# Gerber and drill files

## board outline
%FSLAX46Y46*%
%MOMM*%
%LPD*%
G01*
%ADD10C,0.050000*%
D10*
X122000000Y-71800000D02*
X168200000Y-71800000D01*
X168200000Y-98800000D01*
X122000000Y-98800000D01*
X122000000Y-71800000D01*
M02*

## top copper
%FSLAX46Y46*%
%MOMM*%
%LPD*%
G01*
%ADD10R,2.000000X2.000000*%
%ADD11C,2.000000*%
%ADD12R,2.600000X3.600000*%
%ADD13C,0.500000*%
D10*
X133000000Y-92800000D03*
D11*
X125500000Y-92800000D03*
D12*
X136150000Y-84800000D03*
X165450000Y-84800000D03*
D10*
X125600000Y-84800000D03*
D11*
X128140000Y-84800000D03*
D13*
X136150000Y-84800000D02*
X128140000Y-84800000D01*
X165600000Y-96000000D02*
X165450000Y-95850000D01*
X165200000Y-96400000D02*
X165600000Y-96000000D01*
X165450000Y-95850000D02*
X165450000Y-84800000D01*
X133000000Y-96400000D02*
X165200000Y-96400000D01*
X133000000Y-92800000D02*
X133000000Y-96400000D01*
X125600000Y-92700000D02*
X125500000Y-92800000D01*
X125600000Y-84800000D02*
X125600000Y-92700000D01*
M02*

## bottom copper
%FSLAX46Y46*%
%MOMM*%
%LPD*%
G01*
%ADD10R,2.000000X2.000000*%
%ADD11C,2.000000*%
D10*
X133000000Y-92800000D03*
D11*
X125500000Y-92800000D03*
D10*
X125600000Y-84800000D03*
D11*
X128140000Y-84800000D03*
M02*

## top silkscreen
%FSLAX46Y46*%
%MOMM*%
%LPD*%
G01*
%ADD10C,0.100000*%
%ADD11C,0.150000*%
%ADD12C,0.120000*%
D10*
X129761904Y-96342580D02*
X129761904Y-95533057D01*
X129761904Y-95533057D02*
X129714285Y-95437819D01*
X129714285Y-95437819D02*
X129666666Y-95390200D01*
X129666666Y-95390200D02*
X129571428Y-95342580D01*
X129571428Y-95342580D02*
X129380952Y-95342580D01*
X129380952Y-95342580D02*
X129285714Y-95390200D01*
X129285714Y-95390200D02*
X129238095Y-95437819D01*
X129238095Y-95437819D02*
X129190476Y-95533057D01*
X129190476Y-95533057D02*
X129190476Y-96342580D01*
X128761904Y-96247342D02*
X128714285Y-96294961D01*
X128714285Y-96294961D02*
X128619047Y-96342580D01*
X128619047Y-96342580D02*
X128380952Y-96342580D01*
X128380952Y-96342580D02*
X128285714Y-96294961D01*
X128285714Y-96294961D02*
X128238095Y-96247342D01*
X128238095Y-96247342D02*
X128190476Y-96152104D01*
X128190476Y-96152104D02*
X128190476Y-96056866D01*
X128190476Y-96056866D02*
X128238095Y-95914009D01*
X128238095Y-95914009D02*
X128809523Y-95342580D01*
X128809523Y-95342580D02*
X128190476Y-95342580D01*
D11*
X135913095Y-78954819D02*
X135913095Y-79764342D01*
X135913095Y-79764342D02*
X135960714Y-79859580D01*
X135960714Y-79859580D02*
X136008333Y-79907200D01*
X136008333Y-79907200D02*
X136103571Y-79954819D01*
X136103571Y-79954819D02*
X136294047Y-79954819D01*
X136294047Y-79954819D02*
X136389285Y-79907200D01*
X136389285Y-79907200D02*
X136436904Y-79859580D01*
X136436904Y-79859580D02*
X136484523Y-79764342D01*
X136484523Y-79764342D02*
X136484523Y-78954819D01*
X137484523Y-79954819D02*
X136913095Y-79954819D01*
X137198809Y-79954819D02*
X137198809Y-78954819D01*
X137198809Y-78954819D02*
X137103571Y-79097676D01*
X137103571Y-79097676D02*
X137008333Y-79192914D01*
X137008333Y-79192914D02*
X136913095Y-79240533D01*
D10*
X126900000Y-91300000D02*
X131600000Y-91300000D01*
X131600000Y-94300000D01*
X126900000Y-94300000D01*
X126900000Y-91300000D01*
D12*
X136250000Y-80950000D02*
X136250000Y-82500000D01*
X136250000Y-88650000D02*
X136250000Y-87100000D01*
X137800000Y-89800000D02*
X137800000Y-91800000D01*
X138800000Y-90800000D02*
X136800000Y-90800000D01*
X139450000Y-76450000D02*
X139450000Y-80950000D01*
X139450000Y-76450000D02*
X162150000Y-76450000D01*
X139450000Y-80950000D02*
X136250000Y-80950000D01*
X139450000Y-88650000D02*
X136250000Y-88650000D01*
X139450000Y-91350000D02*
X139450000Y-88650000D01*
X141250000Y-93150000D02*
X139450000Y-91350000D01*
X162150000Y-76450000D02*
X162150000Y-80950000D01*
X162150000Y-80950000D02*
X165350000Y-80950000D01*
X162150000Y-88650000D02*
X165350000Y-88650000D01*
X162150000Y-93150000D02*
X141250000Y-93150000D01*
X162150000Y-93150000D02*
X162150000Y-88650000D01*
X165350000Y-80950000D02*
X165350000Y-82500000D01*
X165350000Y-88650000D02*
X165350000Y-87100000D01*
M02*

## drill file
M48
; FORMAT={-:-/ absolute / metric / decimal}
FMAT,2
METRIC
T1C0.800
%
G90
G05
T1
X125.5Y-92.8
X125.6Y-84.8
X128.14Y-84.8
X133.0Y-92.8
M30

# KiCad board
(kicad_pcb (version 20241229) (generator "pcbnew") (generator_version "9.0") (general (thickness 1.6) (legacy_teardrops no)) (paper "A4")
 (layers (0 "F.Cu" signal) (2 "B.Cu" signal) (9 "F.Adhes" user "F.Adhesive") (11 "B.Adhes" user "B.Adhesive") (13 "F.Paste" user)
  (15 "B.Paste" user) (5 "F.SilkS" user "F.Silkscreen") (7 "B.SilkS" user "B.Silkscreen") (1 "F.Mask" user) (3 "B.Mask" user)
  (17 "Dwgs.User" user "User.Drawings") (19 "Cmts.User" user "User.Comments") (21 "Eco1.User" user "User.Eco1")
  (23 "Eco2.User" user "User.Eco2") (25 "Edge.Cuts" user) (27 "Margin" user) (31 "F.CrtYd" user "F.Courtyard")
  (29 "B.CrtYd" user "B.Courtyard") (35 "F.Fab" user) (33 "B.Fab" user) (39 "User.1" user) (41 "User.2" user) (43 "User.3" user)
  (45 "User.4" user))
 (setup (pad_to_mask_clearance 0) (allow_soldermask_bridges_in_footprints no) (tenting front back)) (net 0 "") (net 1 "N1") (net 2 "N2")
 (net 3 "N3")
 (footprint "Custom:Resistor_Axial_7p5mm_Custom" (layer "F.Cu") (at 133 92.8 180)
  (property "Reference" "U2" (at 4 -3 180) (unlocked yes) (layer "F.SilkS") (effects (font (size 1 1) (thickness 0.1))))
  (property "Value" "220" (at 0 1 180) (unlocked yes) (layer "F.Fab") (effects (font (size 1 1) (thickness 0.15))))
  (fp_rect (start 1.4 -1.5) (end 6.1 1.5) (stroke (width 0.1) (type solid)) (fill no) (layer "F.SilkS"))
  (pad "1" thru_hole rect (at 0 0 180) (size 2 2) (drill 0.8) (layers "*.Cu" "*.Mask") (remove_unused_layers no) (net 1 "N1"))
  (pad "2" thru_hole circle (at 7.5 0 180) (size 2 2) (drill 0.8) (layers "*.Cu" "*.Mask") (remove_unused_layers no) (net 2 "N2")))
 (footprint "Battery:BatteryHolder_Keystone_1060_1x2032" (layer "F.Cu") (at 150.8 84.8)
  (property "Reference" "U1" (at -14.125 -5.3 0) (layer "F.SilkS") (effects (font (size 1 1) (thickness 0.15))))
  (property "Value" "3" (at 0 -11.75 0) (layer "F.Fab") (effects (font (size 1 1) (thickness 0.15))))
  (fp_line (start -14.55 -3.85) (end -14.55 -2.3) (stroke (width 0.12) (type solid)) (layer "F.SilkS"))
  (fp_line (start -14.55 3.85) (end -14.55 2.3) (stroke (width 0.12) (type solid)) (layer "F.SilkS"))
  (fp_line (start -13 5) (end -13 7) (stroke (width 0.12) (type solid)) (layer "F.SilkS"))
  (fp_line (start -12 6) (end -14 6) (stroke (width 0.12) (type solid)) (layer "F.SilkS"))
  (fp_line (start -11.35 -8.35) (end -11.35 -3.85) (stroke (width 0.12) (type solid)) (layer "F.SilkS"))
  (fp_line (start -11.35 -8.35) (end 11.35 -8.35) (stroke (width 0.12) (type solid)) (layer "F.SilkS"))
  (fp_line (start -11.35 -3.85) (end -14.55 -3.85) (stroke (width 0.12) (type solid)) (layer "F.SilkS"))
  (fp_line (start -11.35 3.85) (end -14.55 3.85) (stroke (width 0.12) (type solid)) (layer "F.SilkS"))
  (fp_line (start -11.35 6.55) (end -11.35 3.85) (stroke (width 0.12) (type solid)) (layer "F.SilkS"))
  (fp_line (start -9.55 8.35) (end -11.35 6.55) (stroke (width 0.12) (type solid)) (layer "F.SilkS"))
  (fp_line (start 11.35 -8.35) (end 11.35 -3.85) (stroke (width 0.12) (type solid)) (layer "F.SilkS"))
  (fp_line (start 11.35 -3.85) (end 14.55 -3.85) (stroke (width 0.12) (type solid)) (layer "F.SilkS"))
  (fp_line (start 11.35 3.85) (end 14.55 3.85) (stroke (width 0.12) (type solid)) (layer "F.SilkS"))
  (fp_line (start 11.35 8.35) (end -9.55 8.35) (stroke (width 0.12) (type solid)) (layer "F.SilkS"))
  (fp_line (start 11.35 8.35) (end 11.35 3.85) (stroke (width 0.12) (type solid)) (layer "F.SilkS"))
  (fp_line (start 14.55 -3.85) (end 14.55 -2.3) (stroke (width 0.12) (type solid)) (layer "F.SilkS"))
  (fp_line (start 14.55 3.85) (end 14.55 2.3) (stroke (width 0.12) (type solid)) (layer "F.SilkS"))
  (pad "1" smd rect (at -14.65 0 180) (size 2.6 3.6) (layers "F.Cu" "F.Mask" "F.Paste") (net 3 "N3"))
  (pad "2" smd rect (at 14.65 0 180) (size 2.6 3.6) (layers "F.Cu" "F.Mask" "F.Paste") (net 1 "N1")))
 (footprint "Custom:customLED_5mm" (layer "B.Cu") (at 125.6 84.8)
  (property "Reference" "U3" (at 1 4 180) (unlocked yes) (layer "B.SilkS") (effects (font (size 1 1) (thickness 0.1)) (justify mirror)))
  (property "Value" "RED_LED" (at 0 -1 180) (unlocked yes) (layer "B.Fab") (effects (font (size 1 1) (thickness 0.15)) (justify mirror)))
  (pad "1" thru_hole rect (at 0 0) (size 2 2) (drill 0.8) (layers "*.Cu" "*.Mask") (remove_unused_layers no) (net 2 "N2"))
  (pad "2" thru_hole circle (at 2.54 0) (size 2 2) (drill 0.8) (layers "*.Cu" "*.Mask") (remove_unused_layers no) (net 3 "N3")))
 (gr_rect (start 122 71.8) (end 168.2 98.8) (stroke (width 0.05) (type default)) (fill no) (layer "Edge.Cuts"))
 (segment (start 136.15 84.8) (end 128.14 84.8) (width 0.5) (layer "F.Cu") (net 3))
 (segment (start 165.6 96) (end 165.45 95.85) (width 0.5) (layer "F.Cu") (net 1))
 (segment (start 165.2 96.4) (end 165.6 96) (width 0.5) (layer "F.Cu") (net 1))
 (segment (start 165.45 95.85) (end 165.45 84.8) (width 0.5) (layer "F.Cu") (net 1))
 (segment (start 133 96.4) (end 165.2 96.4) (width 0.5) (layer "F.Cu") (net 1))
 (segment (start 133 92.8) (end 133 96.4) (width 0.5) (layer "F.Cu") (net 1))
 (segment (start 125.6 92.7) (end 125.5 92.8) (width 0.5) (layer "F.Cu") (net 2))
 (segment (start 125.6 84.8) (end 125.6 92.7) (width 0.5) (layer "F.Cu") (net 2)))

